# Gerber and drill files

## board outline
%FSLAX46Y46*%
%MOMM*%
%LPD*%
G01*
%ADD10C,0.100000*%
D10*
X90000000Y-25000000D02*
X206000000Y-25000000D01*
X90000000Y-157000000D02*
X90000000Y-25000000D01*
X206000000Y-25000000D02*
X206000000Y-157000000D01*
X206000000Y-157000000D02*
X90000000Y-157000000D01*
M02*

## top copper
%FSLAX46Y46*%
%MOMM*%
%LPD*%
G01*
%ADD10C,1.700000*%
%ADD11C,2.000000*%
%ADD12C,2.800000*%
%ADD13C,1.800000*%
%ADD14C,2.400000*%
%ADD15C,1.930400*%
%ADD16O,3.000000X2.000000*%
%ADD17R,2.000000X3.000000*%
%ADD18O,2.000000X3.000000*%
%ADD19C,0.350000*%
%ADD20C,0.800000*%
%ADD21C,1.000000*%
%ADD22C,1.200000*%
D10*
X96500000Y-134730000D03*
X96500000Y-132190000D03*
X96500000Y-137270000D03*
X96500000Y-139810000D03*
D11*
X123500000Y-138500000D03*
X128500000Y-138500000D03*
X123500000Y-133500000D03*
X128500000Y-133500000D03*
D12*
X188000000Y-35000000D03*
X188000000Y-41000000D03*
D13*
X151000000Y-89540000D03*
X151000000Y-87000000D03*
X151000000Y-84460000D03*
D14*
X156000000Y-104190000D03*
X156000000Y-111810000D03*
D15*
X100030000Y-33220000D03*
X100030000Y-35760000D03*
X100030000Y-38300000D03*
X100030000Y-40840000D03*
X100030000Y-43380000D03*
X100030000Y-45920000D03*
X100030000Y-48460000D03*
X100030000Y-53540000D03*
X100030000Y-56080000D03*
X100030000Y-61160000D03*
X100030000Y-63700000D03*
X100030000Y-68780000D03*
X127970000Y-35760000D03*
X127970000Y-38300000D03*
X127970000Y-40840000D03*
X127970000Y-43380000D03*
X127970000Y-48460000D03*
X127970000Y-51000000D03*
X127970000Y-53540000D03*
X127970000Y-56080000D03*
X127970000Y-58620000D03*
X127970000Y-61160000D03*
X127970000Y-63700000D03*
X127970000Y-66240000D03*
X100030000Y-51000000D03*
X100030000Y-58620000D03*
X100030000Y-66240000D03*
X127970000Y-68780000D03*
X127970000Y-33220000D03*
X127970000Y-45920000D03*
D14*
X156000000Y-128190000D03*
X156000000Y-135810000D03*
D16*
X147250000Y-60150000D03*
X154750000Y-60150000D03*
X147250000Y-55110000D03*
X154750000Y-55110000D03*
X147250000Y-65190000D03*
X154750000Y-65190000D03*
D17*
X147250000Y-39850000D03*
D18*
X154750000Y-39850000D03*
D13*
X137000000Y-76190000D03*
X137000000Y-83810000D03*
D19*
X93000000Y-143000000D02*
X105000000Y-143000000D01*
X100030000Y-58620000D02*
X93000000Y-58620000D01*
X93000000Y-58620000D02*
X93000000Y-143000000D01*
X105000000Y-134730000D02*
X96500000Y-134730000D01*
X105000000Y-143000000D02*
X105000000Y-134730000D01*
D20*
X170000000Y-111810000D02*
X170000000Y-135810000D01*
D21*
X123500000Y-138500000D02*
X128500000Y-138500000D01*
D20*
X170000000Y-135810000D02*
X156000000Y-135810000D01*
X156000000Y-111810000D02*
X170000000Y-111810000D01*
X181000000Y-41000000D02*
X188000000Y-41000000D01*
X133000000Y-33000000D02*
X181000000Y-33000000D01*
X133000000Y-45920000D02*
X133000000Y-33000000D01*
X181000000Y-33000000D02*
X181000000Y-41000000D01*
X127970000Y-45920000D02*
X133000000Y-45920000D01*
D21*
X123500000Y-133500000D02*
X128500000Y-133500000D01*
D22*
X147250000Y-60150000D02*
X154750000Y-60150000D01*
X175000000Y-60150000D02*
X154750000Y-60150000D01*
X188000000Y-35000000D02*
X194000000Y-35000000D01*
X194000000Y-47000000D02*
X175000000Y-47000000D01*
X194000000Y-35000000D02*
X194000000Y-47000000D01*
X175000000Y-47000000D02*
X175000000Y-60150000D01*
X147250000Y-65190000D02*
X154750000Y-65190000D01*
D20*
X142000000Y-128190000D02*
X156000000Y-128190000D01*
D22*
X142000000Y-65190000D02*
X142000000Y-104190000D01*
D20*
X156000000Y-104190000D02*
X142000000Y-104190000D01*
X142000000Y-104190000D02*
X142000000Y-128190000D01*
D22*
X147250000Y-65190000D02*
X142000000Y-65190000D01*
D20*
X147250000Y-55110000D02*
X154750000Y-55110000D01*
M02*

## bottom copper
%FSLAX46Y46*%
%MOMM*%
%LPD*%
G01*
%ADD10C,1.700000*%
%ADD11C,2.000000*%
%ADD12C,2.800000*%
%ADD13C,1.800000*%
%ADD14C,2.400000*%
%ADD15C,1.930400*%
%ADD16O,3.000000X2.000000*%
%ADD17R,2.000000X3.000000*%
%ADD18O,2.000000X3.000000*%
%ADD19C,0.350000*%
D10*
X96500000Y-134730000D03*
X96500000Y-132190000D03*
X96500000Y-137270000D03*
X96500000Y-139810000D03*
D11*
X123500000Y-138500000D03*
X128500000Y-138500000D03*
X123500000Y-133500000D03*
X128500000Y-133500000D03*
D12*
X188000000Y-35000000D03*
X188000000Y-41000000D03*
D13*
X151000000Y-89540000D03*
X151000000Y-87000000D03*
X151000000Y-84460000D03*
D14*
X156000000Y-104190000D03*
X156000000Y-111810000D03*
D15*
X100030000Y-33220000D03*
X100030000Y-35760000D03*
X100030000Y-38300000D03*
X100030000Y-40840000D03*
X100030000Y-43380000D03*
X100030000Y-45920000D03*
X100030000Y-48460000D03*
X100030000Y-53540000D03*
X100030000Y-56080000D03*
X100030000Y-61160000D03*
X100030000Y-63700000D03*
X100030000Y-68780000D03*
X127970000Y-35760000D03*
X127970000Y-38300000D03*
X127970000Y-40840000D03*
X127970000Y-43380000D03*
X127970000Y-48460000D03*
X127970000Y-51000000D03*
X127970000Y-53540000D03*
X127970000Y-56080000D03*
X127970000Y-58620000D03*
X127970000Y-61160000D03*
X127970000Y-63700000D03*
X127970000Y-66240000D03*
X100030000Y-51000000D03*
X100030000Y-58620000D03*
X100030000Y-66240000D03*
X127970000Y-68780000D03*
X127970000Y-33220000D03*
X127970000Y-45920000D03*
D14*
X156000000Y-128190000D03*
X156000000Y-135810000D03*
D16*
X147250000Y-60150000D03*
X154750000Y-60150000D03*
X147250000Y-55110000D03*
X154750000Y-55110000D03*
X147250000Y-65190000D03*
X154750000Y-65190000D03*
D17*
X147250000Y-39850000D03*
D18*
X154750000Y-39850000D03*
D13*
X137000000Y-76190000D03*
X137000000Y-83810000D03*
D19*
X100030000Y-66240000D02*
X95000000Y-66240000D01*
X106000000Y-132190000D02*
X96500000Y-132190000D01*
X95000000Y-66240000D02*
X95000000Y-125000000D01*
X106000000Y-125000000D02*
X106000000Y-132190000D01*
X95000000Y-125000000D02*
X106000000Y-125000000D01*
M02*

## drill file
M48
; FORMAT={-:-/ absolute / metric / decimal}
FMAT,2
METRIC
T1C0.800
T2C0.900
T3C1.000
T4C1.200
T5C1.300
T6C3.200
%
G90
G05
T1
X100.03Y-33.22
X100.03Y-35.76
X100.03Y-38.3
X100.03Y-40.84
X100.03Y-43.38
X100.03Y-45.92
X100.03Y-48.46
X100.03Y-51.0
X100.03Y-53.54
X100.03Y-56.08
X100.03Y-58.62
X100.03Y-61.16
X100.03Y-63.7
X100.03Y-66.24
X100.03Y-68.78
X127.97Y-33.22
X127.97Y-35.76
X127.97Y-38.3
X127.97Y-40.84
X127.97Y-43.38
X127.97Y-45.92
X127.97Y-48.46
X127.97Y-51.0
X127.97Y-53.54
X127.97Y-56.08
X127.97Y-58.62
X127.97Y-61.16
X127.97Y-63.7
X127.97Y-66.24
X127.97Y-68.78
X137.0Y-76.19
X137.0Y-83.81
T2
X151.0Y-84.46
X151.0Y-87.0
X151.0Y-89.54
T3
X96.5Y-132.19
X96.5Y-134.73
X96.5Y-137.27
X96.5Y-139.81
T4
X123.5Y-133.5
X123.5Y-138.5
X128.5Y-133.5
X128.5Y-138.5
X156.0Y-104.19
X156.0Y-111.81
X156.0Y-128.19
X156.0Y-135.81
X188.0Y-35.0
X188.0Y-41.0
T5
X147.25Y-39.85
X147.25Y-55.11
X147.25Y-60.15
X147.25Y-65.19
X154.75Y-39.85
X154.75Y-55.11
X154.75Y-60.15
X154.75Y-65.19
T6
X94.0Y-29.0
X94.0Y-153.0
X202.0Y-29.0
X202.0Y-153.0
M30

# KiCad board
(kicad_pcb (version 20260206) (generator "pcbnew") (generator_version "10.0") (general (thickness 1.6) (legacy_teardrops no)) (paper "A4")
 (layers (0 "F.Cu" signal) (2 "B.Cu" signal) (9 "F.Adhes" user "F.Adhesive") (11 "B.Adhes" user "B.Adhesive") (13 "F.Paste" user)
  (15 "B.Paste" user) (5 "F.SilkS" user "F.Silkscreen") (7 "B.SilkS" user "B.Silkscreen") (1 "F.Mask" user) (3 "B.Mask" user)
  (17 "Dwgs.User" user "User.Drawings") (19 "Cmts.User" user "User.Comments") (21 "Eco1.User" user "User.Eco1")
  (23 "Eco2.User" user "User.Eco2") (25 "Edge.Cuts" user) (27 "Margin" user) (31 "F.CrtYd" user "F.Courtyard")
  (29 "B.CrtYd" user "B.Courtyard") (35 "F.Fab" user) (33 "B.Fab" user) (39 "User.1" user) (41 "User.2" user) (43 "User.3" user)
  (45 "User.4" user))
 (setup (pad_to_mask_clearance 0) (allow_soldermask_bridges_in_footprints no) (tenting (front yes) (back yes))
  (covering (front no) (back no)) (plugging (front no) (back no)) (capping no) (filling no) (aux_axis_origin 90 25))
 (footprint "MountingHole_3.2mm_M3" (layer "F.Cu") (at 202 153)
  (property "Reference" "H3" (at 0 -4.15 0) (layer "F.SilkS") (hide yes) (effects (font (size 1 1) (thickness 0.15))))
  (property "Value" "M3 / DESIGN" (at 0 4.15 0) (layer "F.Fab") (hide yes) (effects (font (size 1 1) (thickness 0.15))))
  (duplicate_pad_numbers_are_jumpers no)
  (pad "" np_thru_hole circle (at 0 0) (size 3.2 3.2) (drill 3.2) (layers "*.Cu" "*.Mask")))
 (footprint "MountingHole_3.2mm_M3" (layer "F.Cu") (at 94 153)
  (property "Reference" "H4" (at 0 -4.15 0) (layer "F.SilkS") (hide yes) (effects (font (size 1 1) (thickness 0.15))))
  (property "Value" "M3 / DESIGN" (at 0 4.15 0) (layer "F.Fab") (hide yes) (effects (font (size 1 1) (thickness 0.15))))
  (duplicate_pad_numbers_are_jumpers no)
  (pad "" np_thru_hole circle (at 0 0) (size 3.2 3.2) (drill 3.2) (layers "*.Cu" "*.Mask")))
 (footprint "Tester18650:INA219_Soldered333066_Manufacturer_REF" (layer "F.Cu") (at 114 136)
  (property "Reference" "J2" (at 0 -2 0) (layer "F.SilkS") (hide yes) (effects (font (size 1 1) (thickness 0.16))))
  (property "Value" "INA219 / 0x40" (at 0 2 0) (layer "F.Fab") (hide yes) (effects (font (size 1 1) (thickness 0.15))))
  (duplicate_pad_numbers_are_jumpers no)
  (pad "1" thru_hole circle (at -17.5 -1.27) (size 1.7 1.7) (drill 1) (layers "*.Cu" "*.Mask") (remove_unused_layers no)
   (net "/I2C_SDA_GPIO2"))
  (pad "2" thru_hole circle (at -17.5 -3.81) (size 1.7 1.7) (drill 1) (layers "*.Cu" "*.Mask") (remove_unused_layers no)
   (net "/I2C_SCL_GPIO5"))
  (pad "3" thru_hole circle (at -17.5 1.27) (size 1.7 1.7) (drill 1) (layers "*.Cu" "*.Mask") (remove_unused_layers no)
   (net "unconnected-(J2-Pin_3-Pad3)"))
  (pad "4" thru_hole circle (at -17.5 3.81) (size 1.7 1.7) (drill 1) (layers "*.Cu" "*.Mask") (remove_unused_layers no)
   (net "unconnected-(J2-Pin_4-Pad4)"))
  (pad "5" thru_hole circle (at 9.5 2.5) (size 2 2) (drill 1.2) (layers "*.Cu" "*.Mask") (remove_unused_layers no) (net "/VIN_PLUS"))
  (pad "5" thru_hole circle (at 14.5 2.5) (size 2 2) (drill 1.2) (layers "*.Cu" "*.Mask") (remove_unused_layers no) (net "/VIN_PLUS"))
  (pad "6" thru_hole circle (at 9.5 -2.5) (size 2 2) (drill 1.2) (layers "*.Cu" "*.Mask") (remove_unused_layers no) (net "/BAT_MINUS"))
  (pad "6" thru_hole circle (at 14.5 -2.5) (size 2 2) (drill 1.2) (layers "*.Cu" "*.Mask") (remove_unused_layers no) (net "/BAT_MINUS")))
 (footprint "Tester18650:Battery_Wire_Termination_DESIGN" (layer "F.Cu") (at 188 35)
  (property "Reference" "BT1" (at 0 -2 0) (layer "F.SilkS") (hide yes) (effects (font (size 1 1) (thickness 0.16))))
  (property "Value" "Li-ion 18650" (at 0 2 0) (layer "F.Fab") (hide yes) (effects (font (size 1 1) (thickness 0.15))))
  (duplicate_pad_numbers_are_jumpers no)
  (pad "1" thru_hole circle (at 0 0) (size 2.8 2.8) (drill 1.2) (layers "*.Cu" "*.Mask") (remove_unused_layers no) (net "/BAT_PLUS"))
  (pad "2" thru_hole circle (at 0 6) (size 2.8 2.8) (drill 1.2) (layers "*.Cu" "*.Mask") (remove_unused_layers no) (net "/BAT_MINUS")))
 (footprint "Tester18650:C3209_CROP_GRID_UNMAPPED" (layer "F.Cu") (at 151 87)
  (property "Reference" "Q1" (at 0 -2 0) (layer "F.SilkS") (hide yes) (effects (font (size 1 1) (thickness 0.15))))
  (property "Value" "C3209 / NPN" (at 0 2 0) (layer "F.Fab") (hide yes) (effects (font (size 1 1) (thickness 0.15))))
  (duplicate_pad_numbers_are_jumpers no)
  (pad "BOT_B_REF" thru_hole circle (at 0 2.54) (size 1.8 1.8) (drill 0.9) (layers "*.Cu" "*.Mask") (remove_unused_layers no))
  (pad "MID_C_REF" thru_hole circle (at 0 0) (size 1.8 1.8) (drill 0.9) (layers "*.Cu" "*.Mask") (remove_unused_layers no))
  (pad "TOP_E_REF" thru_hole circle (at 0 -2.54) (size 1.8 1.8) (drill 0.9) (layers "*.Cu" "*.Mask") (remove_unused_layers no)))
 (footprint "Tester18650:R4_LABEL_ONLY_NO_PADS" (layer "F.Cu") (at 137 92)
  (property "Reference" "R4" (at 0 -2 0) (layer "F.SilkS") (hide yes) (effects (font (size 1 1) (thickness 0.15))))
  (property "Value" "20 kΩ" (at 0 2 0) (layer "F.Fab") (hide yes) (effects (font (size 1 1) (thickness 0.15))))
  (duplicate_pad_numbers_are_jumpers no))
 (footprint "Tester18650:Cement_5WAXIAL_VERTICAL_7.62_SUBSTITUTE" (layer "F.Cu") (at 156 108)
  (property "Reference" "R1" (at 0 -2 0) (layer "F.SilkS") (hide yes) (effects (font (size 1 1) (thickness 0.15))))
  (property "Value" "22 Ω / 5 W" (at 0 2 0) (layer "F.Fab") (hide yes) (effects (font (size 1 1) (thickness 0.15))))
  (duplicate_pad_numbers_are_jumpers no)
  (pad "1" thru_hole circle (at 0 -3.81) (size 2.4 2.4) (drill 1.2) (layers "*.Cu" "*.Mask") (remove_unused_layers no) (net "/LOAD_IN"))
  (pad "2" thru_hole circle (at 0 3.81) (size 2.4 2.4) (drill 1.2) (layers "*.Cu" "*.Mask") (remove_unused_layers no) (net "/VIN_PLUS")))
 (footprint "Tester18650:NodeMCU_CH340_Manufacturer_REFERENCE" (layer "F.Cu") (at 114 51)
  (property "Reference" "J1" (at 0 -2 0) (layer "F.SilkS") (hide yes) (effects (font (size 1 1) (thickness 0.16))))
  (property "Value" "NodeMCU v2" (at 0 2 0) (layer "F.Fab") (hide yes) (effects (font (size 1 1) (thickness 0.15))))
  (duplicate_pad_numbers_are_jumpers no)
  (pad "" thru_hole circle (at -13.97 -17.78) (size 1.9304 1.9304) (drill 0.8) (layers "*.Cu" "*.Mask") (remove_unused_layers no))
  (pad "" thru_hole circle (at -13.97 -15.24) (size 1.9304 1.9304) (drill 0.8) (layers "*.Cu" "*.Mask") (remove_unused_layers no))
  (pad "" thru_hole circle (at -13.97 -12.7) (size 1.9304 1.9304) (drill 0.8) (layers "*.Cu" "*.Mask") (remove_unused_layers no))
  (pad "" thru_hole circle (at -13.97 -10.16) (size 1.9304 1.9304) (drill 0.8) (layers "*.Cu" "*.Mask") (remove_unused_layers no))
  (pad "" thru_hole circle (at -13.97 -7.62) (size 1.9304 1.9304) (drill 0.8) (layers "*.Cu" "*.Mask") (remove_unused_layers no))
  (pad "" thru_hole circle (at -13.97 -5.08) (size 1.9304 1.9304) (drill 0.8) (layers "*.Cu" "*.Mask") (remove_unused_layers no))
  (pad "" thru_hole circle (at -13.97 -2.54) (size 1.9304 1.9304) (drill 0.8) (layers "*.Cu" "*.Mask") (remove_unused_layers no))
  (pad "" thru_hole circle (at -13.97 2.54) (size 1.9304 1.9304) (drill 0.8) (layers "*.Cu" "*.Mask") (remove_unused_layers no))
  (pad "" thru_hole circle (at -13.97 5.08) (size 1.9304 1.9304) (drill 0.8) (layers "*.Cu" "*.Mask") (remove_unused_layers no))
  (pad "" thru_hole circle (at -13.97 10.16) (size 1.9304 1.9304) (drill 0.8) (layers "*.Cu" "*.Mask") (remove_unused_layers no))
  (pad "" thru_hole circle (at -13.97 12.7) (size 1.9304 1.9304) (drill 0.8) (layers "*.Cu" "*.Mask") (remove_unused_layers no))
  (pad "" thru_hole circle (at -13.97 17.78) (size 1.9304 1.9304) (drill 0.8) (layers "*.Cu" "*.Mask") (remove_unused_layers no))
  (pad "" thru_hole circle (at 13.97 -15.24) (size 1.9304 1.9304) (drill 0.8) (layers "*.Cu" "*.Mask") (remove_unused_layers no))
  (pad "" thru_hole circle (at 13.97 -12.7) (size 1.9304 1.9304) (drill 0.8) (layers "*.Cu" "*.Mask") (remove_unused_layers no))
  (pad "" thru_hole circle (at 13.97 -10.16) (size 1.9304 1.9304) (drill 0.8) (layers "*.Cu" "*.Mask") (remove_unused_layers no))
  (pad "" thru_hole circle (at 13.97 -7.62) (size 1.9304 1.9304) (drill 0.8) (layers "*.Cu" "*.Mask") (remove_unused_layers no))
  (pad "" thru_hole circle (at 13.97 -2.54) (size 1.9304 1.9304) (drill 0.8) (layers "*.Cu" "*.Mask") (remove_unused_layers no))
  (pad "" thru_hole circle (at 13.97 0) (size 1.9304 1.9304) (drill 0.8) (layers "*.Cu" "*.Mask") (remove_unused_layers no))
  (pad "" thru_hole circle (at 13.97 2.54) (size 1.9304 1.9304) (drill 0.8) (layers "*.Cu" "*.Mask") (remove_unused_layers no))
  (pad "" thru_hole circle (at 13.97 5.08) (size 1.9304 1.9304) (drill 0.8) (layers "*.Cu" "*.Mask") (remove_unused_layers no))
  (pad "" thru_hole circle (at 13.97 7.62) (size 1.9304 1.9304) (drill 0.8) (layers "*.Cu" "*.Mask") (remove_unused_layers no))
  (pad "" thru_hole circle (at 13.97 10.16) (size 1.9304 1.9304) (drill 0.8) (layers "*.Cu" "*.Mask") (remove_unused_layers no))
  (pad "" thru_hole circle (at 13.97 12.7) (size 1.9304 1.9304) (drill 0.8) (layers "*.Cu" "*.Mask") (remove_unused_layers no))
  (pad "" thru_hole circle (at 13.97 15.24) (size 1.9304 1.9304) (drill 0.8) (layers "*.Cu" "*.Mask") (remove_unused_layers no))
  (pad "1" thru_hole circle (at -13.97 0) (size 1.9304 1.9304) (drill 0.8) (layers "*.Cu" "*.Mask") (remove_unused_layers no)
   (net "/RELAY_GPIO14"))
  (pad "2" thru_hole circle (at -13.97 7.62) (size 1.9304 1.9304) (drill 0.8) (layers "*.Cu" "*.Mask") (remove_unused_layers no)
   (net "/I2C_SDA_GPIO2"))
  (pad "3" thru_hole circle (at -13.97 15.24) (size 1.9304 1.9304) (drill 0.8) (layers "*.Cu" "*.Mask") (remove_unused_layers no)
   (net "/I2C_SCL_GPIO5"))
  (pad "4" thru_hole circle (at 13.97 17.78) (size 1.9304 1.9304) (drill 0.8) (layers "*.Cu" "*.Mask") (remove_unused_layers no)
   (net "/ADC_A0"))
  (pad "5" thru_hole circle (at 13.97 -17.78) (size 1.9304 1.9304) (drill 0.8) (layers "*.Cu" "*.Mask") (remove_unused_layers no)
   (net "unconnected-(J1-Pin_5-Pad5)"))
  (pad "6" thru_hole circle (at 13.97 -5.08) (size 1.9304 1.9304) (drill 0.8) (layers "*.Cu" "*.Mask") (remove_unused_layers no)
   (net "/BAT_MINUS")))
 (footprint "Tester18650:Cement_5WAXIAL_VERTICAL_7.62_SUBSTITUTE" (layer "F.Cu") (at 156 132)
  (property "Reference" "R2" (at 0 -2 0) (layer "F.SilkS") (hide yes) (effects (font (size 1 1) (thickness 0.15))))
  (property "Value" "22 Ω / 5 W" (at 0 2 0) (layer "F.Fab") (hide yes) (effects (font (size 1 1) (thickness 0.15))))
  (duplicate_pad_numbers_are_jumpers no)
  (pad "1" thru_hole circle (at 0 -3.81) (size 2.4 2.4) (drill 1.2) (layers "*.Cu" "*.Mask") (remove_unused_layers no) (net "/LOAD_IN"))
  (pad "2" thru_hole circle (at 0 3.81) (size 2.4 2.4) (drill 1.2) (layers "*.Cu" "*.Mask") (remove_unused_layers no) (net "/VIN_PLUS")))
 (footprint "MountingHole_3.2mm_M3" (layer "F.Cu") (at 202 29)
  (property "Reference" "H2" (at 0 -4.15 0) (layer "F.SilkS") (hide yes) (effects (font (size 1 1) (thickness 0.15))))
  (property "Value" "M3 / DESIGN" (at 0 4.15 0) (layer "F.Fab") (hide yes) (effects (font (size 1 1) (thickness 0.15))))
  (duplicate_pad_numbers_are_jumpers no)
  (pad "" np_thru_hole circle (at 0 0) (size 3.2 3.2) (drill 3.2) (layers "*.Cu" "*.Mask")))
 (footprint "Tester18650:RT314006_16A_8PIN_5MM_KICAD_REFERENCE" (layer "F.Cu") (at 151 52)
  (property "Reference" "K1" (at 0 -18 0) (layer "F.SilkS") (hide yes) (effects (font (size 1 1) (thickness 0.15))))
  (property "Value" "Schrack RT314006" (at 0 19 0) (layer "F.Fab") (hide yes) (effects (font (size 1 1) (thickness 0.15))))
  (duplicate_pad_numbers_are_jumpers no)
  (pad "11" thru_hole oval (at -3.75 8.15) (size 3 2) (drill 1.3) (layers "*.Cu" "*.Mask") (remove_unused_layers no) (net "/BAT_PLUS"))
  (pad "11" thru_hole oval (at 3.75 8.15) (size 3 2) (drill 1.3) (layers "*.Cu" "*.Mask") (remove_unused_layers no) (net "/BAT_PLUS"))
  (pad "12" thru_hole oval (at -3.75 3.11) (size 3 2) (drill 1.3) (layers "*.Cu" "*.Mask") (remove_unused_layers no)
   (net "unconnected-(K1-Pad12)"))
  (pad "12" thru_hole oval (at 3.75 3.11) (size 3 2) (drill 1.3) (layers "*.Cu" "*.Mask") (remove_unused_layers no)
   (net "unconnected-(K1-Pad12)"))
  (pad "14" thru_hole oval (at -3.75 13.19) (size 3 2) (drill 1.3) (layers "*.Cu" "*.Mask") (remove_unused_layers no) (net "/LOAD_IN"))
  (pad "14" thru_hole oval (at 3.75 13.19) (size 3 2) (drill 1.3) (layers "*.Cu" "*.Mask") (remove_unused_layers no) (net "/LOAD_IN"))
  (pad "A1" thru_hole rect (at -3.75 -12.15) (size 2 3) (drill 1.3) (layers "*.Cu" "*.Mask") (remove_unused_layers no) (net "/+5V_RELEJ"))
  (pad "A2" thru_hole oval (at 3.75 -12.15) (size 2 3) (drill 1.3) (layers "*.Cu" "*.Mask") (remove_unused_layers no) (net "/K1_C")))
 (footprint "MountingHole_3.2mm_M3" (layer "F.Cu") (at 94 29)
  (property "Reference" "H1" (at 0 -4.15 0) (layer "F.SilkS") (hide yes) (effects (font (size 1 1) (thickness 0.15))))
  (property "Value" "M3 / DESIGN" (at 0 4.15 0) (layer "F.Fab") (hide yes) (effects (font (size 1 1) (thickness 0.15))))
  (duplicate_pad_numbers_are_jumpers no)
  (pad "" np_thru_hole circle (at 0 0) (size 3.2 3.2) (drill 3.2) (layers "*.Cu" "*.Mask")))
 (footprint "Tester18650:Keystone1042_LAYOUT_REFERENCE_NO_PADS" (layer "F.Cu") (at 190 95)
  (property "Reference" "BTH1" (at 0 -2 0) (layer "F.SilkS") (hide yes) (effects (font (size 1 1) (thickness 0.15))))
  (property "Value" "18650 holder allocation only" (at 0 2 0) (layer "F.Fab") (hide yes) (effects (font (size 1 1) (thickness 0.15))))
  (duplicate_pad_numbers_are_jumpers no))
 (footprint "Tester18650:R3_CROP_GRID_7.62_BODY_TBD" (layer "F.Cu") (at 137 80)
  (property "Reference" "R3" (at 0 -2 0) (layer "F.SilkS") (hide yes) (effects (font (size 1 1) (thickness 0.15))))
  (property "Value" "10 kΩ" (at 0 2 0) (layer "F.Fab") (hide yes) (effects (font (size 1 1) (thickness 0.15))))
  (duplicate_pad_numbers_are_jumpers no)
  (pad "1" thru_hole circle (at 0 -3.81) (size 1.8 1.8) (drill 0.8) (layers "*.Cu" "*.Mask") (remove_unused_layers no)
   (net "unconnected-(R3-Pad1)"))
  (pad "2" thru_hole circle (at 0 3.81) (size 1.8 1.8) (drill 0.8) (layers "*.Cu" "*.Mask") (remove_unused_layers no)
   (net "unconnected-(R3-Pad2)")))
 (gr_line (start 90 25) (end 206 25) (stroke (width 0.1) (type default)) (layer "Edge.Cuts"))
 (gr_line (start 90 157) (end 90 25) (stroke (width 0.1) (type default)) (layer "Edge.Cuts"))
 (gr_line (start 206 25) (end 206 157) (stroke (width 0.1) (type default)) (layer "Edge.Cuts"))
 (gr_line (start 206 157) (end 90 157) (stroke (width 0.1) (type default)) (layer "Edge.Cuts"))
 (segment (start 93 143) (end 105 143) (width 0.35) (layer "F.Cu") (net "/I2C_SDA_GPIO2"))
 (segment (start 100.03 58.62) (end 93 58.62) (width 0.35) (layer "F.Cu") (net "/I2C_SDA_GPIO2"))
 (segment (start 93 58.62) (end 93 143) (width 0.35) (layer "F.Cu") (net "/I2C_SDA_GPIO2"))
 (segment (start 105 134.73) (end 96.5 134.73) (width 0.35) (layer "F.Cu") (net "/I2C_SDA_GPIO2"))
 (segment (start 105 143) (end 105 134.73) (width 0.35) (layer "F.Cu") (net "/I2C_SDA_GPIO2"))
 (segment (start 100.03 66.24) (end 95 66.24) (width 0.35) (layer "B.Cu") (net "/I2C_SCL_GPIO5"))
 (segment (start 106 132.19) (end 96.5 132.19) (width 0.35) (layer "B.Cu") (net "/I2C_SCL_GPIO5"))
 (segment (start 95 66.24) (end 95 125) (width 0.35) (layer "B.Cu") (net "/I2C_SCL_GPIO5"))
 (segment (start 106 125) (end 106 132.19) (width 0.35) (layer "B.Cu") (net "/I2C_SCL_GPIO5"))
 (segment (start 95 125) (end 106 125) (width 0.35) (layer "B.Cu") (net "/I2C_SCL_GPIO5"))
 (segment (start 170 111.81) (end 170 135.81) (width 0.8) (layer "F.Cu") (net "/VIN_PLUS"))
 (segment (start 123.5 138.5) (end 128.5 138.5) (width 1) (layer "F.Cu") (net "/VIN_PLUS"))
 (segment (start 170 135.81) (end 156 135.81) (width 0.8) (layer "F.Cu") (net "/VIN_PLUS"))
 (segment (start 156 111.81) (end 170 111.81) (width 0.8) (layer "F.Cu") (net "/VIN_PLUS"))
 (segment (start 181 41) (end 188 41) (width 0.8) (layer "F.Cu") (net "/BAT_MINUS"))
 (segment (start 133 33) (end 181 33) (width 0.8) (layer "F.Cu") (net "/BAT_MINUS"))
 (segment (start 133 45.92) (end 133 33) (width 0.8) (layer "F.Cu") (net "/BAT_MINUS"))
 (segment (start 181 33) (end 181 41) (width 0.8) (layer "F.Cu") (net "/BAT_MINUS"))
 (segment (start 127.97 45.92) (end 133 45.92) (width 0.8) (layer "F.Cu") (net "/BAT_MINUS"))
 (segment (start 123.5 133.5) (end 128.5 133.5) (width 1) (layer "F.Cu") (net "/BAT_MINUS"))
 (segment (start 147.25 60.15) (end 154.75 60.15) (width 1.2) (layer "F.Cu") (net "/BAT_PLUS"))
 (segment (start 175 60.15) (end 154.75 60.15) (width 1.2) (layer "F.Cu") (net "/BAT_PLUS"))
 (segment (start 188 35) (end 194 35) (width 1.2) (layer "F.Cu") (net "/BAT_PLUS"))
 (segment (start 194 47) (end 175 47) (width 1.2) (layer "F.Cu") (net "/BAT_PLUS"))
 (segment (start 194 35) (end 194 47) (width 1.2) (layer "F.Cu") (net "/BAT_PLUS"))
 (segment (start 175 47) (end 175 60.15) (width 1.2) (layer "F.Cu") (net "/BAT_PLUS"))
 (segment (start 147.25 65.19) (end 154.75 65.19) (width 1.2) (layer "F.Cu") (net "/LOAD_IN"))
 (segment (start 142 128.19) (end 156 128.19) (width 0.8) (layer "F.Cu") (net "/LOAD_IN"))
 (segment (start 142 65.19) (end 142 104.19) (width 1.2) (layer "F.Cu") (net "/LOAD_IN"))
 (segment (start 156 104.19) (end 142 104.19) (width 0.8) (layer "F.Cu") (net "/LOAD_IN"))
 (segment (start 142 104.19) (end 142 128.19) (width 0.8) (layer "F.Cu") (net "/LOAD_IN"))
 (segment (start 147.25 65.19) (end 142 65.19) (width 1.2) (layer "F.Cu") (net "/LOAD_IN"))
 (segment (start 147.25 55.11) (end 154.75 55.11) (width 0.8) (layer "F.Cu") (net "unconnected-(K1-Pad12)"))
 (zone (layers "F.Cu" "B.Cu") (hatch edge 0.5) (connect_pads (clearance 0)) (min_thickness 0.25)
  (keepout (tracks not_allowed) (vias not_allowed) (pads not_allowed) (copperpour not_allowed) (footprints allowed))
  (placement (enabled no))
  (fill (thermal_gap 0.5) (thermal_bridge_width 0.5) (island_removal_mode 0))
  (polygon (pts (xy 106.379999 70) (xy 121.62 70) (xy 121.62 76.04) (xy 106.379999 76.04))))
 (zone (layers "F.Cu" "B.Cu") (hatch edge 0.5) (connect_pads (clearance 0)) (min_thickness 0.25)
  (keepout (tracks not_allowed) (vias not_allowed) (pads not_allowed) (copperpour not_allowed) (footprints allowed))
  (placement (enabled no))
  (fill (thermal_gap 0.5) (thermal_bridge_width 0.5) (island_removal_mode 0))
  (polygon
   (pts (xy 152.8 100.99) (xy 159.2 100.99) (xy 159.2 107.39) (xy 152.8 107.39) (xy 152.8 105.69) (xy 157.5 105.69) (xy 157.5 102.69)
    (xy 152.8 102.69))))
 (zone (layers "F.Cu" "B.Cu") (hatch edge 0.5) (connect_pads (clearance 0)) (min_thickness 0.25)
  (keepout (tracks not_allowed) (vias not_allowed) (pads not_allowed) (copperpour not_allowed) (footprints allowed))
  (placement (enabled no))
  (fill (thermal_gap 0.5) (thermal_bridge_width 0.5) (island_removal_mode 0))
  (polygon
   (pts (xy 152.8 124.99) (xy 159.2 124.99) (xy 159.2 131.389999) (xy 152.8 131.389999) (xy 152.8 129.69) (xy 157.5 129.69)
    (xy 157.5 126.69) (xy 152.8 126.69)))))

